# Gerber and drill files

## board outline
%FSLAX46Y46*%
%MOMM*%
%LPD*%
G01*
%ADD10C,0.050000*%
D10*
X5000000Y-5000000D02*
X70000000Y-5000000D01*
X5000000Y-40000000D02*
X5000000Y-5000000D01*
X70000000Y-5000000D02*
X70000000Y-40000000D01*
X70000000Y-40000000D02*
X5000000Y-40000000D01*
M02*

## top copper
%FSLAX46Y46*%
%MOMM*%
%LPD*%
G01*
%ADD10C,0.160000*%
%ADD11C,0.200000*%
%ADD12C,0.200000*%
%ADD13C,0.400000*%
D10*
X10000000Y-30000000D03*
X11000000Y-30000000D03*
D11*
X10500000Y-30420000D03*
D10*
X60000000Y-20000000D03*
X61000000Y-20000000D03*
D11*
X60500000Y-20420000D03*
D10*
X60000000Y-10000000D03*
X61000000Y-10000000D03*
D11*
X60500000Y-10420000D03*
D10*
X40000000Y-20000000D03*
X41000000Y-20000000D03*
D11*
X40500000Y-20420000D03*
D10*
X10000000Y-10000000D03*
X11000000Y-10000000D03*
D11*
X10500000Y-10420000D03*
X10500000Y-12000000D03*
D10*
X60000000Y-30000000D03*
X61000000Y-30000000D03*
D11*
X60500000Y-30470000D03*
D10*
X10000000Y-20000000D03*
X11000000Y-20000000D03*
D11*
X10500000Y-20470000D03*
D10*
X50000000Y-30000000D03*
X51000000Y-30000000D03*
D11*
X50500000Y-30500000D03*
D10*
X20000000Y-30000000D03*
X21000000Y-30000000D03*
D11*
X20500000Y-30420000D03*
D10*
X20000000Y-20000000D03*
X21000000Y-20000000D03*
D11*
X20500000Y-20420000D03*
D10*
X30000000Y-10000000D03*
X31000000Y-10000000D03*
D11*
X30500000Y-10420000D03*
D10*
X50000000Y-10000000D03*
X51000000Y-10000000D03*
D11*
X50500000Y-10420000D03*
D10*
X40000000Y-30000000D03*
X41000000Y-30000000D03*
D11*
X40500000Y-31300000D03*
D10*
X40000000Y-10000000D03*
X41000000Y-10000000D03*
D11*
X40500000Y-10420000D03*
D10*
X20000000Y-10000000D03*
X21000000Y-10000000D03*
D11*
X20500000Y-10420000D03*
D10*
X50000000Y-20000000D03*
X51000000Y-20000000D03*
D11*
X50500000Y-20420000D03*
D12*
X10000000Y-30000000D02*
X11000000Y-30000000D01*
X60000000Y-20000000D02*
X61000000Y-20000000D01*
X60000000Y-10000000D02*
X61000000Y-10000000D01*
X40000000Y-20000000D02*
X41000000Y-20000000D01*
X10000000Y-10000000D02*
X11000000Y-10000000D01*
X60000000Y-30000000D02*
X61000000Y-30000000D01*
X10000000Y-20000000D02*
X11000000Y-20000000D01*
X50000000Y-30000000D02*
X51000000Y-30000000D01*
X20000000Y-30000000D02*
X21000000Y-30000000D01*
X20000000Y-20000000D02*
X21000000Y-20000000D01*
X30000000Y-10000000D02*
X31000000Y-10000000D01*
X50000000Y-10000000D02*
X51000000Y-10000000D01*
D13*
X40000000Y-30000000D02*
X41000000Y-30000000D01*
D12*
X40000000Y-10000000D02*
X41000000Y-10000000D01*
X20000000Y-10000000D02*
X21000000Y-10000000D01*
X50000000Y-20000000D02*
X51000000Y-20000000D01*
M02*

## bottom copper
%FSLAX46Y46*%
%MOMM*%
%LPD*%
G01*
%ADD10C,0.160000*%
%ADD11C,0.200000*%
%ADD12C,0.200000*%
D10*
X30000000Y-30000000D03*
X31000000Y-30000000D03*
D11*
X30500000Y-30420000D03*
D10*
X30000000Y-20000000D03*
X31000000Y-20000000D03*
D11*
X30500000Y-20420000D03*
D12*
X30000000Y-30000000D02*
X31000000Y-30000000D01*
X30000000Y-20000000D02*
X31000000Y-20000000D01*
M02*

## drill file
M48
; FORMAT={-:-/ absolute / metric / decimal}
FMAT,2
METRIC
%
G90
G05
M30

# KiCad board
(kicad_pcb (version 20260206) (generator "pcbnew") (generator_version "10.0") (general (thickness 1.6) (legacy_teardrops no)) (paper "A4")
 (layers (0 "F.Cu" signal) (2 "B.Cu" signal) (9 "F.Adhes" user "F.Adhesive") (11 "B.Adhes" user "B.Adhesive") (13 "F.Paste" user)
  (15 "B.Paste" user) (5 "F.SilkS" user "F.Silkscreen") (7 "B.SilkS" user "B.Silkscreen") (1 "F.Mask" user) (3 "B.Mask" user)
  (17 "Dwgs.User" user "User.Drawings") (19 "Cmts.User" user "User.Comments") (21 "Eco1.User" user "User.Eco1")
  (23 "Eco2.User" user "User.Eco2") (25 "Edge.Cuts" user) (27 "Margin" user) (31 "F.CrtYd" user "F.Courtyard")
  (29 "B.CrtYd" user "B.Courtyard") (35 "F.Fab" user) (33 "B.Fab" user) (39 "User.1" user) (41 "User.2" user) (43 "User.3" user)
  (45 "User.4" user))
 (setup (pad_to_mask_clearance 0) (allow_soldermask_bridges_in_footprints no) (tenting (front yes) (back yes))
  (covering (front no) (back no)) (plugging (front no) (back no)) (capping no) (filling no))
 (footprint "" (layer "F.Cu") (at 10 30)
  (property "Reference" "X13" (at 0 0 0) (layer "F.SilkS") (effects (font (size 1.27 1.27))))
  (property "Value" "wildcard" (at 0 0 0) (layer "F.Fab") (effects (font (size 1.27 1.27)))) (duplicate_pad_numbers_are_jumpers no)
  (pad "1" smd circle (at 0 0) (size 0.16 0.16) (layers "F.Cu") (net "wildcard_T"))
  (pad "2" smd circle (at 1 0) (size 0.16 0.16) (layers "F.Cu") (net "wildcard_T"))
  (pad "3" smd circle (at 0.5 0.42) (size 0.2 0.2) (layers "F.Cu") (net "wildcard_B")))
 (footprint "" (layer "F.Cu") (at 60 20)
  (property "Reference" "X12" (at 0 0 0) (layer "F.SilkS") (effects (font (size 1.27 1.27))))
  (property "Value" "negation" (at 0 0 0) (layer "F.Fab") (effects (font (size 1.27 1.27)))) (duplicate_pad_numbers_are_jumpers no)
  (pad "1" smd circle (at 0 0) (size 0.16 0.16) (layers "F.Cu") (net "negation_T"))
  (pad "2" smd circle (at 1 0) (size 0.16 0.16) (layers "F.Cu") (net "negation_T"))
  (pad "3" smd circle (at 0.5 0.42) (size 0.2 0.2) (layers "F.Cu") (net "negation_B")))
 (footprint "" (layer "F.Cu") (at 60 10)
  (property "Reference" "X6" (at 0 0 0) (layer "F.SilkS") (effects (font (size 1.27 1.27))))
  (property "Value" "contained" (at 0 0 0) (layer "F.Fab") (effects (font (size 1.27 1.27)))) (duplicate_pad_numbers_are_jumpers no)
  (pad "1" smd circle (at 0 0) (size 0.16 0.16) (layers "F.Cu") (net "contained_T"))
  (pad "2" smd circle (at 1 0) (size 0.16 0.16) (layers "F.Cu") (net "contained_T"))
  (pad "3" smd circle (at 0.5 0.42) (size 0.2 0.2) (layers "F.Cu") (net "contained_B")))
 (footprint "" (layer "F.Cu") (at 40 20)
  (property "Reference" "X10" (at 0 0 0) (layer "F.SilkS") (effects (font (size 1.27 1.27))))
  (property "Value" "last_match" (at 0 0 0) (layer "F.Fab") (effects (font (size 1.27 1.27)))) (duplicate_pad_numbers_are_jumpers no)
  (pad "1" smd circle (at 0 0) (size 0.16 0.16) (layers "F.Cu") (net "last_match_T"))
  (pad "2" smd circle (at 1 0) (size 0.16 0.16) (layers "F.Cu") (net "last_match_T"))
  (pad "3" smd circle (at 0.5 0.42) (size 0.2 0.2) (layers "F.Cu") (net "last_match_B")))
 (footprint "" (layer "F.Cu") (at 10 10)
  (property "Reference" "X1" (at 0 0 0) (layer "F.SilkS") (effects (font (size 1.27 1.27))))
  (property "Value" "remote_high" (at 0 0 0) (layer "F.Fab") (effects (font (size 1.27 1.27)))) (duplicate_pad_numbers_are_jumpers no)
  (pad "1" smd circle (at 0 0) (size 0.16 0.16) (layers "F.Cu") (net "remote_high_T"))
  (pad "2" smd circle (at 1 0) (size 0.16 0.16) (layers "F.Cu") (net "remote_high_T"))
  (pad "3" smd circle (at 0.5 0.42) (size 0.2 0.2) (layers "F.Cu") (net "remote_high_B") (clearance 0.15))
  (pad "4" smd circle (at 0.5 2) (size 0.2 0.2) (layers "F.Cu") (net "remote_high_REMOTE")))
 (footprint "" (layer "F.Cu") (at 60 30)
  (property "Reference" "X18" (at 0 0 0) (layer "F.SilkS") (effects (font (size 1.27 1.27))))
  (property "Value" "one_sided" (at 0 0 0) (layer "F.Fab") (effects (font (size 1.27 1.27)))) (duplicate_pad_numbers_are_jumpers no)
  (pad "1" smd circle (at 0 0) (size 0.16 0.16) (layers "F.Cu") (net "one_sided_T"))
  (pad "2" smd circle (at 1 0) (size 0.16 0.16) (layers "F.Cu") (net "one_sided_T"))
  (pad "3" smd circle (at 0.5 0.47) (size 0.2 0.2) (layers "F.Cu") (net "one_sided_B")))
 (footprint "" (layer "F.Cu") (at 10 20)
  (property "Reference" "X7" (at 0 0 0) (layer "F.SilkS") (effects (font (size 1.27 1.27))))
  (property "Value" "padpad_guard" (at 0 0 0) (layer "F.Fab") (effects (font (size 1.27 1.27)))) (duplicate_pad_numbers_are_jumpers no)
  (pad "1" smd circle (at 0 0) (size 0.16 0.16) (layers "F.Cu") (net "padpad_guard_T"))
  (pad "2" smd circle (at 1 0) (size 0.16 0.16) (layers "F.Cu") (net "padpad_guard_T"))
  (pad "3" smd circle (at 0.5 0.47) (size 0.2 0.2) (layers "F.Cu") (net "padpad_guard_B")))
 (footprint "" (layer "F.Cu") (at 50 30)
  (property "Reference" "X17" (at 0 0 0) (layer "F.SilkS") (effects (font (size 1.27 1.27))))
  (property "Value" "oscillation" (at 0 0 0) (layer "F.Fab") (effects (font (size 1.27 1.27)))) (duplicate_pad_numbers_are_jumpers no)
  (pad "1" smd circle (at 0 0) (size 0.16 0.16) (layers "F.Cu") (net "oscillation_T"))
  (pad "2" smd circle (at 1 0) (size 0.16 0.16) (layers "F.Cu") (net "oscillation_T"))
  (pad "3" smd circle (at 0.5 0.5) (size 0.2 0.2) (layers "F.Cu") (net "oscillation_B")))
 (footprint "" (layer "F.Cu") (at 20 30)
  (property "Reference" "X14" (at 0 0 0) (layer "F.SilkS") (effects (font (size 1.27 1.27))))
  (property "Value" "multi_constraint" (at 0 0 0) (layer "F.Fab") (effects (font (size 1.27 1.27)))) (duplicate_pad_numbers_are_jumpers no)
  (pad "1" smd circle (at 0 0) (size 0.16 0.16) (layers "F.Cu") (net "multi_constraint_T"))
  (pad "2" smd circle (at 1 0) (size 0.16 0.16) (layers "F.Cu") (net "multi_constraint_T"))
  (pad "3" smd circle (at 0.5 0.42) (size 0.2 0.2) (layers "F.Cu") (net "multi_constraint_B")))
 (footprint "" (layer "F.Cu") (at 30 30)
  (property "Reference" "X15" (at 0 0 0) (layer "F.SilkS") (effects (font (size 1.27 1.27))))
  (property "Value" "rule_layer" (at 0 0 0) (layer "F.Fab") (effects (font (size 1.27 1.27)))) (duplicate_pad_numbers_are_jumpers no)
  (pad "1" smd circle (at 0 0) (size 0.16 0.16) (layers "B.Cu") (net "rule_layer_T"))
  (pad "2" smd circle (at 1 0) (size 0.16 0.16) (layers "B.Cu") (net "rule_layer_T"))
  (pad "3" smd circle (at 0.5 0.42) (size 0.2 0.2) (layers "B.Cu") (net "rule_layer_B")))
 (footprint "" (layer "F.Cu") (at 20 20)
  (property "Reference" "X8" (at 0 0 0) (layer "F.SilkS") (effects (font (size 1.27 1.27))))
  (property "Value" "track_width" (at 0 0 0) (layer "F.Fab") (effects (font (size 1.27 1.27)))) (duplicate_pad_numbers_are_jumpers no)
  (pad "1" smd circle (at 0 0) (size 0.16 0.16) (layers "F.Cu") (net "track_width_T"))
  (pad "2" smd circle (at 1 0) (size 0.16 0.16) (layers "F.Cu") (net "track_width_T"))
  (pad "3" smd circle (at 0.5 0.42) (size 0.2 0.2) (layers "F.Cu") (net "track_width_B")))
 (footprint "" (layer "F.Cu") (at 30 10)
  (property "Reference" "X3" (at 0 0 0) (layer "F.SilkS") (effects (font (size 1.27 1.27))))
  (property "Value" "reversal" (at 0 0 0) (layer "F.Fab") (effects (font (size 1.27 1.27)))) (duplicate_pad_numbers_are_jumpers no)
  (pad "1" smd circle (at 0 0) (size 0.16 0.16) (layers "F.Cu") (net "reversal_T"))
  (pad "2" smd circle (at 1 0) (size 0.16 0.16) (layers "F.Cu") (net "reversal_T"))
  (pad "3" smd circle (at 0.5 0.42) (size 0.2 0.2) (layers "F.Cu") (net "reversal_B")))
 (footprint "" (layer "F.Cu") (at 50 10)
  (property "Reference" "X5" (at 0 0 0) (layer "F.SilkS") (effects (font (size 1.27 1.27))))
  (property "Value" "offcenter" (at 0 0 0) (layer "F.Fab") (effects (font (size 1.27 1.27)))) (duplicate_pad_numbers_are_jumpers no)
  (pad "1" smd circle (at 0 0) (size 0.16 0.16) (layers "F.Cu") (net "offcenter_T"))
  (pad "2" smd circle (at 1 0) (size 0.16 0.16) (layers "F.Cu") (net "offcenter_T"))
  (pad "3" smd circle (at 0.5 0.42) (size 0.2 0.2) (layers "F.Cu") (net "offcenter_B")))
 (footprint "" (layer "F.Cu") (at 40 30)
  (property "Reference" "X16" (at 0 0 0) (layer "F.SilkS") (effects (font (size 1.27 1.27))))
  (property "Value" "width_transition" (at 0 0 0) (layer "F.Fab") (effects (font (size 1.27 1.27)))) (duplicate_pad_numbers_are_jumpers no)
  (pad "1" smd circle (at 0 0) (size 0.16 0.16) (layers "F.Cu") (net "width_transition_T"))
  (pad "2" smd circle (at 1 0) (size 0.16 0.16) (layers "F.Cu") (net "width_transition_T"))
  (pad "3" smd circle (at 0.5 1.3) (size 0.2 0.2) (layers "F.Cu") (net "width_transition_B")))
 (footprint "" (layer "F.Cu") (at 30 20)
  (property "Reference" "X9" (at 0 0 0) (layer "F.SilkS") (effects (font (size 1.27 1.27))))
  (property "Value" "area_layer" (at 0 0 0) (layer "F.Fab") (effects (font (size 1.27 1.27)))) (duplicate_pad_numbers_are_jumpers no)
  (pad "1" smd circle (at 0 0) (size 0.16 0.16) (layers "B.Cu") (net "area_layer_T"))
  (pad "2" smd circle (at 1 0) (size 0.16 0.16) (layers "B.Cu") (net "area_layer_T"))
  (pad "3" smd circle (at 0.5 0.42) (size 0.2 0.2) (layers "B.Cu") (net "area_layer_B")))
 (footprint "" (layer "F.Cu") (at 40 10)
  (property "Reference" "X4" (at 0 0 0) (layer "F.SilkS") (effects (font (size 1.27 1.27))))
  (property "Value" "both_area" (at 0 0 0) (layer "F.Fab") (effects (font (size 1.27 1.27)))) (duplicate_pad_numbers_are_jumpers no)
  (pad "1" smd circle (at 0 0) (size 0.16 0.16) (layers "F.Cu") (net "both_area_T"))
  (pad "2" smd circle (at 1 0) (size 0.16 0.16) (layers "F.Cu") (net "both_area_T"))
  (pad "3" smd circle (at 0.5 0.42) (size 0.2 0.2) (layers "F.Cu") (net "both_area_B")))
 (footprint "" (layer "F.Cu") (at 20 10)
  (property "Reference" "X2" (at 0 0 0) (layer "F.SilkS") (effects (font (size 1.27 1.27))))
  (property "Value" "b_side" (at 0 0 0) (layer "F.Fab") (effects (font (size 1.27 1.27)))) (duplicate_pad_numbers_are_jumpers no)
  (pad "1" smd circle (at 0 0) (size 0.16 0.16) (layers "F.Cu") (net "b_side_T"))
  (pad "2" smd circle (at 1 0) (size 0.16 0.16) (layers "F.Cu") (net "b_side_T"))
  (pad "3" smd circle (at 0.5 0.42) (size 0.2 0.2) (layers "F.Cu") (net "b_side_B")))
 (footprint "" (layer "F.Cu") (at 50 20)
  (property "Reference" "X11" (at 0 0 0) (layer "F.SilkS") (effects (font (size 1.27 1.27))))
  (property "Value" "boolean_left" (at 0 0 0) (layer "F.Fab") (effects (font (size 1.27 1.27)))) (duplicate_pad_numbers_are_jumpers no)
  (pad "1" smd circle (at 0 0) (size 0.16 0.16) (layers "F.Cu") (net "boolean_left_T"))
  (pad "2" smd circle (at 1 0) (size 0.16 0.16) (layers "F.Cu") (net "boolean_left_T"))
  (pad "3" smd circle (at 0.5 0.42) (size 0.2 0.2) (layers "F.Cu") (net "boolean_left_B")))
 (gr_line (start 5 5) (end 70 5) (stroke (width 0.05) (type default)) (layer "Edge.Cuts"))
 (gr_line (start 5 40) (end 5 5) (stroke (width 0.05) (type default)) (layer "Edge.Cuts"))
 (gr_line (start 70 5) (end 70 40) (stroke (width 0.05) (type default)) (layer "Edge.Cuts"))
 (gr_line (start 70 40) (end 5 40) (stroke (width 0.05) (type default)) (layer "Edge.Cuts"))
 (segment (start 10 30) (end 11 30) (width 0.2) (layer "F.Cu") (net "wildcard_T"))
 (segment (start 60 20) (end 61 20) (width 0.2) (layer "F.Cu") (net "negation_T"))
 (segment (start 60 10) (end 61 10) (width 0.2) (layer "F.Cu") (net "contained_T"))
 (segment (start 40 20) (end 41 20) (width 0.2) (layer "F.Cu") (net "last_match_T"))
 (segment (start 10 10) (end 11 10) (width 0.2) (layer "F.Cu") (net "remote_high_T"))
 (segment (start 60 30) (end 61 30) (width 0.2) (layer "F.Cu") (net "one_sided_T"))
 (segment (start 10 20) (end 11 20) (width 0.2) (layer "F.Cu") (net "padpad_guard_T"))
 (segment (start 50 30) (end 51 30) (width 0.2) (layer "F.Cu") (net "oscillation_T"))
 (segment (start 20 30) (end 21 30) (width 0.2) (layer "F.Cu") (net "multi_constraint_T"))
 (segment (start 30 30) (end 31 30) (width 0.2) (layer "B.Cu") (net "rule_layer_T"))
 (segment (start 20 20) (end 21 20) (width 0.2) (layer "F.Cu") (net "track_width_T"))
 (segment (start 30 10) (end 31 10) (width 0.2) (layer "F.Cu") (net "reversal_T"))
 (segment (start 50 10) (end 51 10) (width 0.2) (layer "F.Cu") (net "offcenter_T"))
 (segment (start 40 30) (end 41 30) (width 0.4) (layer "F.Cu") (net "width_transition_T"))
 (segment (start 30 20) (end 31 20) (width 0.2) (layer "B.Cu") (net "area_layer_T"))
 (segment (start 40 10) (end 41 10) (width 0.2) (layer "F.Cu") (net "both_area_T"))
 (segment (start 20 10) (end 21 10) (width 0.2) (layer "F.Cu") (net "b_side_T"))
 (segment (start 50 20) (end 51 20) (width 0.2) (layer "F.Cu") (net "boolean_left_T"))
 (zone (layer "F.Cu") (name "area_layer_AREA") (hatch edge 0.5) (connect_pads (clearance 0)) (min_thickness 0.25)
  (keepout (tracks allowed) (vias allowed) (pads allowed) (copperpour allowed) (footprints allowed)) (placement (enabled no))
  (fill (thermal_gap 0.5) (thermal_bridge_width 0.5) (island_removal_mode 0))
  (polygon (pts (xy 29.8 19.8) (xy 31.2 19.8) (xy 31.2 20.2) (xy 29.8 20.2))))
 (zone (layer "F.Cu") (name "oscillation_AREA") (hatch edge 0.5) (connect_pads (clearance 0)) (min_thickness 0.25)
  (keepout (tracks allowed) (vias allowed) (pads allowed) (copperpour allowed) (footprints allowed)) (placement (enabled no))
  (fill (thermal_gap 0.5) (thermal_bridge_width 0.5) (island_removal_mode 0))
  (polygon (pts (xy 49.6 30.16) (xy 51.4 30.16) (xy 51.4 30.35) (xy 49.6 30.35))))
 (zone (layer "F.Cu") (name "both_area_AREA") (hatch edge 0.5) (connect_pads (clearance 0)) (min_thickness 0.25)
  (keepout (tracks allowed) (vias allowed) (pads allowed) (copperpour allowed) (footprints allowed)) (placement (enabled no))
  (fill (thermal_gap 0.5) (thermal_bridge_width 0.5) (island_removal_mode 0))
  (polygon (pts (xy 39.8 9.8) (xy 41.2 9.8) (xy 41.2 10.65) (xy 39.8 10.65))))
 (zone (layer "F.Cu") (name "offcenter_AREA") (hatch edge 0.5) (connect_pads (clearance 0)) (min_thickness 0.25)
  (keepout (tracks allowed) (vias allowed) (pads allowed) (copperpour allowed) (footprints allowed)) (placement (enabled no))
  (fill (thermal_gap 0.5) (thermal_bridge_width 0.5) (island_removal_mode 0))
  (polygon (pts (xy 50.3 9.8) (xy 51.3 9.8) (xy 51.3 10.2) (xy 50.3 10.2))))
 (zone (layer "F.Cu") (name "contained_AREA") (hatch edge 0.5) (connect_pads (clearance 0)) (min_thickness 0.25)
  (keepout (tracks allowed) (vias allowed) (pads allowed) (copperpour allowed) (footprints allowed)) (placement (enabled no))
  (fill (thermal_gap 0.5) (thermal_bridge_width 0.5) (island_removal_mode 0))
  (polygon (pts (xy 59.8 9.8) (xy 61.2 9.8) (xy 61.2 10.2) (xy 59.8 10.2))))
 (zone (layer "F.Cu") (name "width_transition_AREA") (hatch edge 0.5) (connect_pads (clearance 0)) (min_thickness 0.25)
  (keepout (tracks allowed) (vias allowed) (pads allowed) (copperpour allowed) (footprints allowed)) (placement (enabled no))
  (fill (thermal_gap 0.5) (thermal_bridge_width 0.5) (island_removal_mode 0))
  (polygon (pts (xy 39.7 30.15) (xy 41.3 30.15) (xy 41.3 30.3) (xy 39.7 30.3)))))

